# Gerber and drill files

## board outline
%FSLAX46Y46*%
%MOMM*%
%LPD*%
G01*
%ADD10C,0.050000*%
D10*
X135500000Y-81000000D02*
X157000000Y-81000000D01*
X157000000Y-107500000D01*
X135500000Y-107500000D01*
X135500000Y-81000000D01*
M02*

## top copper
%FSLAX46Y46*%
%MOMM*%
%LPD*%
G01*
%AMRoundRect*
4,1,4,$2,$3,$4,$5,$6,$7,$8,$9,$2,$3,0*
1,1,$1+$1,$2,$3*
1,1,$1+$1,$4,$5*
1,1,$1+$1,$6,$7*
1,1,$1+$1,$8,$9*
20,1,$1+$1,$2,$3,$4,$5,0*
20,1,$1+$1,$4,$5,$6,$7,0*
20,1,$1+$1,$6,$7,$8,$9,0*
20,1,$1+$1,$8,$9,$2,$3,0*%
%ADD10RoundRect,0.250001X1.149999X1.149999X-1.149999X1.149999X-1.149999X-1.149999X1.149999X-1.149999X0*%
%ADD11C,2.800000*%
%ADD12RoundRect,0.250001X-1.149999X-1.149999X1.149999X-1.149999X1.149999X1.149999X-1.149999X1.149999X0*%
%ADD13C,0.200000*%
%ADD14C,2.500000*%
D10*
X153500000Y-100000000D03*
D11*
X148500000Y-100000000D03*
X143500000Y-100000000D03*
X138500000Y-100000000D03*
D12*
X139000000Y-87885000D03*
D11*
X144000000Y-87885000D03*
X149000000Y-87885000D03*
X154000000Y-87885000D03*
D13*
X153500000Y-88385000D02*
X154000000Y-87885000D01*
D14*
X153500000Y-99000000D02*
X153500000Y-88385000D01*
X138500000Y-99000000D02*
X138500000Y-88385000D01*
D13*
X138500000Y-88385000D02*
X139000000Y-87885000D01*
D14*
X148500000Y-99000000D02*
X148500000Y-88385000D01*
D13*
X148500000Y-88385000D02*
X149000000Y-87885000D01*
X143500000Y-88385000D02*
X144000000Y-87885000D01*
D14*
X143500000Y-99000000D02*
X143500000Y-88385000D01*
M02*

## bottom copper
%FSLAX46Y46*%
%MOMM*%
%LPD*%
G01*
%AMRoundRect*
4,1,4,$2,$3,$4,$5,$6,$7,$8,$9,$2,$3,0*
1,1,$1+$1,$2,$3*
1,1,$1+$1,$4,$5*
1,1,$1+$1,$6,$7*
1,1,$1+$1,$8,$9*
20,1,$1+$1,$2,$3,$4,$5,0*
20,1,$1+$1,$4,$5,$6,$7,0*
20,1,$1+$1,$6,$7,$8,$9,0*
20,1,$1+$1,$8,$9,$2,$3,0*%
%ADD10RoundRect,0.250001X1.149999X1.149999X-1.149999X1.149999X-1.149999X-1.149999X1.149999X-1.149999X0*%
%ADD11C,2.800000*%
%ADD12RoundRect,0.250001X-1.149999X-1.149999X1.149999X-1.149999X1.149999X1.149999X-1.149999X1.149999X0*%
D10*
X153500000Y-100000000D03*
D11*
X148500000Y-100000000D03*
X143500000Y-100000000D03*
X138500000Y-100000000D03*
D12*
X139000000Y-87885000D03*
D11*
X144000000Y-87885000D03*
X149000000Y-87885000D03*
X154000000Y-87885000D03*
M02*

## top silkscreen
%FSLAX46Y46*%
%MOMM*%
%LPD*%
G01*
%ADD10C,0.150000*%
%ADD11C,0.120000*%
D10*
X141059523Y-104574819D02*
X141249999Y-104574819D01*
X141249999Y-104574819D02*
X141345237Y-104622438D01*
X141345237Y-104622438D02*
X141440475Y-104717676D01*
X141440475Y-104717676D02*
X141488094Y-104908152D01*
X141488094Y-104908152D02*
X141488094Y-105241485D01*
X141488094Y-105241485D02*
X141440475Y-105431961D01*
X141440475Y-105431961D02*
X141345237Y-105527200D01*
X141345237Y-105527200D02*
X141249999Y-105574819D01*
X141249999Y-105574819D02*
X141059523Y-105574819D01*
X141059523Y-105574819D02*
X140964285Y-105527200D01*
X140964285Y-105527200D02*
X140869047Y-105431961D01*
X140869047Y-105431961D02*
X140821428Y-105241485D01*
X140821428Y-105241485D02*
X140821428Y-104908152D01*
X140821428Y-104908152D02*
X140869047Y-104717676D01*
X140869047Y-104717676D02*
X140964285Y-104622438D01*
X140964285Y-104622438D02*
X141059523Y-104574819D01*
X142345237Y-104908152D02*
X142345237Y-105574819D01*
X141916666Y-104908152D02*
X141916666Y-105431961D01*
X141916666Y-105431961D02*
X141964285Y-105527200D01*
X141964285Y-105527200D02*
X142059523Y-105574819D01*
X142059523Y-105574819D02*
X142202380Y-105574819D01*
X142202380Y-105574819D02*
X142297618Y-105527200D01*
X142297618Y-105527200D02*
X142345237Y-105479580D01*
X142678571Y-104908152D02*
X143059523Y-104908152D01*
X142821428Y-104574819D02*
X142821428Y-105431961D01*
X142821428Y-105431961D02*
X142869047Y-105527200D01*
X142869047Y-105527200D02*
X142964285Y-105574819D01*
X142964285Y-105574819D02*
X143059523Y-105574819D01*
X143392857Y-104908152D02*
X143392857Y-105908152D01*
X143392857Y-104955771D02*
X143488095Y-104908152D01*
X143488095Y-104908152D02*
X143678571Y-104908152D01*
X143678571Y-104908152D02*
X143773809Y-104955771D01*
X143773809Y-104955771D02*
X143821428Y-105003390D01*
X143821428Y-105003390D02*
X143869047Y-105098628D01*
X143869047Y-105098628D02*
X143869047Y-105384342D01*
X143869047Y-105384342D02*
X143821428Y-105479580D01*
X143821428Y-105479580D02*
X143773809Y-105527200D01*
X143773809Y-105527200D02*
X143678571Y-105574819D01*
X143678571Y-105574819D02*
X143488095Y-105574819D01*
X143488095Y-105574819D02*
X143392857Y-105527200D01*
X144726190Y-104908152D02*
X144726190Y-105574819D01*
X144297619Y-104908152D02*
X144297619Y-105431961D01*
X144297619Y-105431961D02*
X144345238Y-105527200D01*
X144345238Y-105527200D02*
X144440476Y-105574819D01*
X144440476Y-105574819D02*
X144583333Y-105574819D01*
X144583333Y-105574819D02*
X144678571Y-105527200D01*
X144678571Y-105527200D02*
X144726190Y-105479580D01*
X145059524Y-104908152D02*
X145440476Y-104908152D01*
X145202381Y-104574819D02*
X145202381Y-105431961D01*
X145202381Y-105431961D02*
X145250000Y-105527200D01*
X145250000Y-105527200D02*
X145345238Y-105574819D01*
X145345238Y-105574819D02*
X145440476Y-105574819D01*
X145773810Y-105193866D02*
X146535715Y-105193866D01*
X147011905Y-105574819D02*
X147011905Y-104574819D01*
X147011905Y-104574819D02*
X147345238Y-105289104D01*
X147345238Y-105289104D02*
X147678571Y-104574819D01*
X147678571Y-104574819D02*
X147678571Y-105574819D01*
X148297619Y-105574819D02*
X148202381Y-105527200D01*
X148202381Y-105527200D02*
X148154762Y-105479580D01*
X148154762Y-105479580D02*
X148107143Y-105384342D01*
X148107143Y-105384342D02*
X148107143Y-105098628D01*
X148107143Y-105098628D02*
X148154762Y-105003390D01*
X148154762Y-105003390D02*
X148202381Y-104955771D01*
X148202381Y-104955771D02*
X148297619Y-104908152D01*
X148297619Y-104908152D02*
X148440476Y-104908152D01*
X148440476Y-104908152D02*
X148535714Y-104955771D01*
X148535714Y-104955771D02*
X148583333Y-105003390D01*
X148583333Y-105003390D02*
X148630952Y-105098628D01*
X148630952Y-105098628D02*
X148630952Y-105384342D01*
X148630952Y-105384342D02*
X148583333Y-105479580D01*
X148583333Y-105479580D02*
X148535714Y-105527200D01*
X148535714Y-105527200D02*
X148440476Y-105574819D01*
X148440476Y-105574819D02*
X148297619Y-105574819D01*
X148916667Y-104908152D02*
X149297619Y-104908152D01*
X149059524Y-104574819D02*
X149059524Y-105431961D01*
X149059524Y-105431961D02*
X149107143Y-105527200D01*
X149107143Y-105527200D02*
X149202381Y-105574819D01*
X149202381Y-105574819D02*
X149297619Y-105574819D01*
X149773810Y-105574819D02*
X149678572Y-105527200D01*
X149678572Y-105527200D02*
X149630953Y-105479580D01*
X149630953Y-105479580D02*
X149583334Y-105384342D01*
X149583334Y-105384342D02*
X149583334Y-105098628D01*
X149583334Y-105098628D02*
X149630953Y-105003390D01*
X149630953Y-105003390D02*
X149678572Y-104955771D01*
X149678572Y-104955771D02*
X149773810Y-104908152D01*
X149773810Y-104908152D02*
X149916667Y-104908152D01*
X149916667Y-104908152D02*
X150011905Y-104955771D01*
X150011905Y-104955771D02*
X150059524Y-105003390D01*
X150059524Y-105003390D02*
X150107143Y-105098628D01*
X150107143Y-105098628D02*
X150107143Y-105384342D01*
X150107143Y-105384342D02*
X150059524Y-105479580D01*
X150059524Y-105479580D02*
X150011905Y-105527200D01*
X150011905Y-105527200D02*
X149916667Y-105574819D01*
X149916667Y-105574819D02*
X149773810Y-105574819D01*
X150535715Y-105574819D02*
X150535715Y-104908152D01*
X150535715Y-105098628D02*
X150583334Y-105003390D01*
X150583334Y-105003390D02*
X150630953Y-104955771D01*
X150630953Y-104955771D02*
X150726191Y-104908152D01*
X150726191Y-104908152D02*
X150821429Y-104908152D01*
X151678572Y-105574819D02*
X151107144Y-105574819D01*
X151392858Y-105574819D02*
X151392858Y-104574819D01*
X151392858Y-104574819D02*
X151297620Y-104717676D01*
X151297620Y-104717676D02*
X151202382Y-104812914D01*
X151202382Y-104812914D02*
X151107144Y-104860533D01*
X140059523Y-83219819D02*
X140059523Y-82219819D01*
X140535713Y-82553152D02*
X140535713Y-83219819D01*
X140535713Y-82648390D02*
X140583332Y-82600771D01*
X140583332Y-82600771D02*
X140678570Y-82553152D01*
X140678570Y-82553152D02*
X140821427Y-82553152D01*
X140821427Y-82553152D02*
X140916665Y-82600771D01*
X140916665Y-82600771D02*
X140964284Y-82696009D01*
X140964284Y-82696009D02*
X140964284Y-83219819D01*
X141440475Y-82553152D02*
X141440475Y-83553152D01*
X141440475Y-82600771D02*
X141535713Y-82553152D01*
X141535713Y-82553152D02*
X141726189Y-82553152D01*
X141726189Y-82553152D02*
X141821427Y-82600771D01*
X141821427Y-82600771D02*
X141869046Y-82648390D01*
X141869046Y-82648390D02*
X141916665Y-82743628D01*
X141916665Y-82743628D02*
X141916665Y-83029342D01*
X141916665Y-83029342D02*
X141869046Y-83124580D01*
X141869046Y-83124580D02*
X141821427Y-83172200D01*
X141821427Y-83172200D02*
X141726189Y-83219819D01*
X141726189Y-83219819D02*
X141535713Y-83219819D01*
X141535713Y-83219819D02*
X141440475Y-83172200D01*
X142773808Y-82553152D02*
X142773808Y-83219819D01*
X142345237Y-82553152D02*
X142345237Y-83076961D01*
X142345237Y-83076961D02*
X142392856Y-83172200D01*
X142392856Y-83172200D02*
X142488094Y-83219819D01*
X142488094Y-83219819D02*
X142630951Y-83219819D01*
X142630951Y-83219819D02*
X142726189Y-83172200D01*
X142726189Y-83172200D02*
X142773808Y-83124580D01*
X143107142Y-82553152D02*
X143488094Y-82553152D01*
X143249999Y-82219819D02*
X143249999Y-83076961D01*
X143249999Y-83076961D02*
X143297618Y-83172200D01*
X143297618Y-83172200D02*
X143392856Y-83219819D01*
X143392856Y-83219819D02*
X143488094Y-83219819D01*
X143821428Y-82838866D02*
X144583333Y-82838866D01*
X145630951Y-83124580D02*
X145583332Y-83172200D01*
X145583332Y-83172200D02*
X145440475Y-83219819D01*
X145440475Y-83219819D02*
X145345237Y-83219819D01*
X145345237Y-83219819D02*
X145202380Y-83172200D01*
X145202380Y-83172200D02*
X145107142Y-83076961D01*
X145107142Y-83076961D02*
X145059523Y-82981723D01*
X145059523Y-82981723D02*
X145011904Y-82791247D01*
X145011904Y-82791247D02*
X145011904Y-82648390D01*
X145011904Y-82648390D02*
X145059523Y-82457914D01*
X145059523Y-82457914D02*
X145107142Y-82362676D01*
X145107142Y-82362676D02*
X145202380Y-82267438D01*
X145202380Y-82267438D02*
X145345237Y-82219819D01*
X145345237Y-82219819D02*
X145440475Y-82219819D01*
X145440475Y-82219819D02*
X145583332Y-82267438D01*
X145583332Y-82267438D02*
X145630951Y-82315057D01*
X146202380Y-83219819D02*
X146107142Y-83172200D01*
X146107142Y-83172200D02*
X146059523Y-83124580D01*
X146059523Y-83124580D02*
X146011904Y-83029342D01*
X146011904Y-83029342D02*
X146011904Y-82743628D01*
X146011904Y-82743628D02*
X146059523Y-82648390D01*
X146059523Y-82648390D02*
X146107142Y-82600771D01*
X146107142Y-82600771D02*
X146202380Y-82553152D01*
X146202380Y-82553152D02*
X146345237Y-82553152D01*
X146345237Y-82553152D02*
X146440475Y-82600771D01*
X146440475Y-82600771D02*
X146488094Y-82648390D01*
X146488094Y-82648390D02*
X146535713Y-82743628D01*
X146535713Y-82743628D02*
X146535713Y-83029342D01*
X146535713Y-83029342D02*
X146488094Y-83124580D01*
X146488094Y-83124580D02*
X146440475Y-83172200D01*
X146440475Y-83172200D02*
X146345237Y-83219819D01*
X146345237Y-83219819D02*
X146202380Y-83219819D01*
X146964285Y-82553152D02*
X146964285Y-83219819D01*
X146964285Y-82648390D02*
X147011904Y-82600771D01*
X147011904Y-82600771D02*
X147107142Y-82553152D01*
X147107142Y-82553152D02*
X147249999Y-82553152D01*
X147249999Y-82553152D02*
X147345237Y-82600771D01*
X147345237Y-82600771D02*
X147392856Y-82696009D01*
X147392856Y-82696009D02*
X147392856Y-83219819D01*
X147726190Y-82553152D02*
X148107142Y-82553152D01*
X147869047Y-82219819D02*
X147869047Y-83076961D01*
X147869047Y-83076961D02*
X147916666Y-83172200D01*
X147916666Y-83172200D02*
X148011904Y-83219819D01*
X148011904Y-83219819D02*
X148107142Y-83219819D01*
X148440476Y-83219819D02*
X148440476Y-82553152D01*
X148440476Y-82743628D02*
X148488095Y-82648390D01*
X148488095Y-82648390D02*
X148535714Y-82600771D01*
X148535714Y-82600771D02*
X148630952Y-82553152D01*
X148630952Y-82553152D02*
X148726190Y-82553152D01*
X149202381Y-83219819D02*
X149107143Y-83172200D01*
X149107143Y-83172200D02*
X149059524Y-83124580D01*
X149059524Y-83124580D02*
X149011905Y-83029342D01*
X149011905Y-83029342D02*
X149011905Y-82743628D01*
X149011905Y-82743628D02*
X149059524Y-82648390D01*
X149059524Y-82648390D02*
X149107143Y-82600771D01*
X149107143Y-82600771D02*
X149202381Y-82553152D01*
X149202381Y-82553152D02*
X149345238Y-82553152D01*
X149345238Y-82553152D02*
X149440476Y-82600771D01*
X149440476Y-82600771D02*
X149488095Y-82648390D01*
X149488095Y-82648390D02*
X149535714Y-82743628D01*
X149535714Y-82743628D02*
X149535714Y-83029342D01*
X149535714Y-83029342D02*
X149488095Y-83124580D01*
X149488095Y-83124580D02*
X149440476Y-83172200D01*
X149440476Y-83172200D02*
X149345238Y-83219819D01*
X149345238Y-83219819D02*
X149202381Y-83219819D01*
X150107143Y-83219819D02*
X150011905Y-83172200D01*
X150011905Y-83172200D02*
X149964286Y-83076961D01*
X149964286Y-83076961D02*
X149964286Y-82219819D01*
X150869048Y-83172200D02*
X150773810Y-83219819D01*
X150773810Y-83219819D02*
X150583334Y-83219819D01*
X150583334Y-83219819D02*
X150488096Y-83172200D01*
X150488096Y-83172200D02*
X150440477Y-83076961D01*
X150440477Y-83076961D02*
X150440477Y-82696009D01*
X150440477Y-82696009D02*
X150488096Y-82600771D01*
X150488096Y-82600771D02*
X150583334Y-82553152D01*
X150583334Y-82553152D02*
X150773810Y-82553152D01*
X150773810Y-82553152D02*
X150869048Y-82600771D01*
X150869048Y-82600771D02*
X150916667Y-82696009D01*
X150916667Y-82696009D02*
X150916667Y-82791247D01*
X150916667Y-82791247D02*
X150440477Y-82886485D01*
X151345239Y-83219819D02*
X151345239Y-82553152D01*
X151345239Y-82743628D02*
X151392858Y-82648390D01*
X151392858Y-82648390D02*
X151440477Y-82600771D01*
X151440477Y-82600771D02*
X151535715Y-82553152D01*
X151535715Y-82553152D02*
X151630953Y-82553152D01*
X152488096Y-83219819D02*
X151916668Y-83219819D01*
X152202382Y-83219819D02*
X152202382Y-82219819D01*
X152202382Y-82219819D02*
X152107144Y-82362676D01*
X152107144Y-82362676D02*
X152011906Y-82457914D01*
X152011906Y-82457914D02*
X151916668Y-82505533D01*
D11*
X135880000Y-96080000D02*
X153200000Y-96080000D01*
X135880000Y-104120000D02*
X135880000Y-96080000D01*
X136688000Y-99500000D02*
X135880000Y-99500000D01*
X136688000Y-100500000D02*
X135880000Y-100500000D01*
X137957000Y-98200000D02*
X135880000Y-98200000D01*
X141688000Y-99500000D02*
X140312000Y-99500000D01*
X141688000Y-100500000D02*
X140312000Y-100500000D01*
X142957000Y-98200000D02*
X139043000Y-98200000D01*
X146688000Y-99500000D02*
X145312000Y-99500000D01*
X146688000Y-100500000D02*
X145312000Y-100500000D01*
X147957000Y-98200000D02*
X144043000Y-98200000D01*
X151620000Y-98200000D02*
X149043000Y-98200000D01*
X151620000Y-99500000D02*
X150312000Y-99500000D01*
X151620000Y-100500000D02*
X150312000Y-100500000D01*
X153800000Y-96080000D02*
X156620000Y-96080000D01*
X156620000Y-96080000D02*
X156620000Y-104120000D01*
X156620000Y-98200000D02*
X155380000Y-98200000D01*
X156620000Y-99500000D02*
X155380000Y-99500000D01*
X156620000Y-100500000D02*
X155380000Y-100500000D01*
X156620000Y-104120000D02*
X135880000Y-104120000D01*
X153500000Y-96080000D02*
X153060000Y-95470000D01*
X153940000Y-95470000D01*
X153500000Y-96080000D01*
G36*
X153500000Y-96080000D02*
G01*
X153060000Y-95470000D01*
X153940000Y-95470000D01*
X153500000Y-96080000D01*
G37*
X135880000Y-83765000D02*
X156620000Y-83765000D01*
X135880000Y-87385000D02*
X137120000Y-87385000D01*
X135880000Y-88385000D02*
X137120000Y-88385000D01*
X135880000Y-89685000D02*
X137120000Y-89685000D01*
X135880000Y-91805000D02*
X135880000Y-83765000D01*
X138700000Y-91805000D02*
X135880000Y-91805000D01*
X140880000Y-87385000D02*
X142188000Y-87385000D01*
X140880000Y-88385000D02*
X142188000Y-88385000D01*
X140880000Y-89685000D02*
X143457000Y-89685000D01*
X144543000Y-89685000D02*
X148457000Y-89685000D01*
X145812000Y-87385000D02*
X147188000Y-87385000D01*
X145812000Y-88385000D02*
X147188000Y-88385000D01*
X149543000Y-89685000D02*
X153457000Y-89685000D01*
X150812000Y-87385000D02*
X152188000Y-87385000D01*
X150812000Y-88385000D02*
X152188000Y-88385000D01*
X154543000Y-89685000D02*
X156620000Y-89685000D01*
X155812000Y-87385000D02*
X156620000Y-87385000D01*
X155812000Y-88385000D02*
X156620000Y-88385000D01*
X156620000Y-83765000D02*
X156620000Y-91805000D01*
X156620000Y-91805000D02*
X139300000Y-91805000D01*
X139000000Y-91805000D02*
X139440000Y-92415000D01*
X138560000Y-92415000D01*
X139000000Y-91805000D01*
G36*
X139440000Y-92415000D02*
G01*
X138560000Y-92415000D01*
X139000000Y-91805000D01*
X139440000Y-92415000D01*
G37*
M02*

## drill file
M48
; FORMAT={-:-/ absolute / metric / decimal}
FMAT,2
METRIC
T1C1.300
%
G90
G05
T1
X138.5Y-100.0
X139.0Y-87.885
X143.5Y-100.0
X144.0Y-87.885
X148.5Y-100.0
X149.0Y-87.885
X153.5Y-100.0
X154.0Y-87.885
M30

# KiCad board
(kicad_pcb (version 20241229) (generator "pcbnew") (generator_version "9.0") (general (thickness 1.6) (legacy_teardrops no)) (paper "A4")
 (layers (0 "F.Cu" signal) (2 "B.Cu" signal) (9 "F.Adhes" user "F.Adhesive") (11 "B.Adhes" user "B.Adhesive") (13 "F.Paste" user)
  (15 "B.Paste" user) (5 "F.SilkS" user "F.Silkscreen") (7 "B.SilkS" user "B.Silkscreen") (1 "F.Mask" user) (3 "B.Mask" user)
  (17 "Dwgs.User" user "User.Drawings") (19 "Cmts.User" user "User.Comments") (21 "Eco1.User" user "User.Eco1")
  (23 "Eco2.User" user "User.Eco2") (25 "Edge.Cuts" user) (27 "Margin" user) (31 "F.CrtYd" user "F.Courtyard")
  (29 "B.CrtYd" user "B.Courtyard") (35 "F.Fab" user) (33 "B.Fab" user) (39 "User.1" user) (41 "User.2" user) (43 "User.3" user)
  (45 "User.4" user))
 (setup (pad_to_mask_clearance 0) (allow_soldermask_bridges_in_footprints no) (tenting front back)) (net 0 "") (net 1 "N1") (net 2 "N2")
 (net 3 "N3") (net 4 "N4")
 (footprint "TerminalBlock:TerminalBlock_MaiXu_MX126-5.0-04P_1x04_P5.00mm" (layer "F.Cu") (at 153.5 100 180)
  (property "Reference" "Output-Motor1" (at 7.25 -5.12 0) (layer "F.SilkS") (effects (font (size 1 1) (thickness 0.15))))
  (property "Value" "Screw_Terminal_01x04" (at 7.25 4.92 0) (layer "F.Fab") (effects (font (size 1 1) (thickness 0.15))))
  (fp_line (start 17.62 3.92) (end 0.3 3.92) (stroke (width 0.12) (type solid)) (layer "F.SilkS"))
  (fp_line (start 17.62 -4.12) (end 17.62 3.92) (stroke (width 0.12) (type solid)) (layer "F.SilkS"))
  (fp_line (start 16.812 0.5) (end 17.62 0.5) (stroke (width 0.12) (type solid)) (layer "F.SilkS"))
  (fp_line (start 16.812 -0.5) (end 17.62 -0.5) (stroke (width 0.12) (type solid)) (layer "F.SilkS"))
  (fp_line (start 15.543 1.8) (end 17.62 1.8) (stroke (width 0.12) (type solid)) (layer "F.SilkS"))
  (fp_line (start 11.812 0.5) (end 13.188 0.5) (stroke (width 0.12) (type solid)) (layer "F.SilkS"))
  (fp_line (start 11.812 -0.5) (end 13.188 -0.5) (stroke (width 0.12) (type solid)) (layer "F.SilkS"))
  (fp_line (start 10.543 1.8) (end 14.457 1.8) (stroke (width 0.12) (type solid)) (layer "F.SilkS"))
  (fp_line (start 6.812 0.5) (end 8.188 0.5) (stroke (width 0.12) (type solid)) (layer "F.SilkS"))
  (fp_line (start 6.812 -0.5) (end 8.188 -0.5) (stroke (width 0.12) (type solid)) (layer "F.SilkS"))
  (fp_line (start 5.543 1.8) (end 9.457 1.8) (stroke (width 0.12) (type solid)) (layer "F.SilkS"))
  (fp_line (start 1.88 1.8) (end 4.457 1.8) (stroke (width 0.12) (type solid)) (layer "F.SilkS"))
  (fp_line (start 1.88 0.5) (end 3.188 0.5) (stroke (width 0.12) (type solid)) (layer "F.SilkS"))
  (fp_line (start 1.88 -0.5) (end 3.188 -0.5) (stroke (width 0.12) (type solid)) (layer "F.SilkS"))
  (fp_line (start -0.3 3.92) (end -3.12 3.92) (stroke (width 0.12) (type solid)) (layer "F.SilkS"))
  (fp_line (start -3.12 3.92) (end -3.12 -4.12) (stroke (width 0.12) (type solid)) (layer "F.SilkS"))
  (fp_line (start -3.12 1.8) (end -1.88 1.8) (stroke (width 0.12) (type solid)) (layer "F.SilkS"))
  (fp_line (start -3.12 0.5) (end -1.88 0.5) (stroke (width 0.12) (type solid)) (layer "F.SilkS"))
  (fp_line (start -3.12 -0.5) (end -1.88 -0.5) (stroke (width 0.12) (type solid)) (layer "F.SilkS"))
  (fp_line (start -3.12 -4.12) (end 17.62 -4.12) (stroke (width 0.12) (type solid)) (layer "F.SilkS"))
  (fp_poly (pts (xy 0 3.92) (xy 0.44 4.53) (xy -0.44 4.53)) (stroke (width 0.12) (type solid)) (fill yes) (layer "F.SilkS"))
  (pad "1" thru_hole roundrect (at 0 0 180) (size 2.8 2.8) (drill 1.3) (layers "*.Cu" "*.Mask") (remove_unused_layers no)
   (roundrect_rratio 0.089286) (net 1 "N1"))
  (pad "2" thru_hole circle (at 5 0 180) (size 2.8 2.8) (drill 1.3) (layers "*.Cu" "*.Mask") (remove_unused_layers no) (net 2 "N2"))
  (pad "3" thru_hole circle (at 10 0 180) (size 2.8 2.8) (drill 1.3) (layers "*.Cu" "*.Mask") (remove_unused_layers no) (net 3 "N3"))
  (pad "4" thru_hole circle (at 15 0 180) (size 2.8 2.8) (drill 1.3) (layers "*.Cu" "*.Mask") (remove_unused_layers no) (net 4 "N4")))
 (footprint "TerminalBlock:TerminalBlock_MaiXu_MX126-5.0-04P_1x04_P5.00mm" (layer "F.Cu") (at 139 87.885)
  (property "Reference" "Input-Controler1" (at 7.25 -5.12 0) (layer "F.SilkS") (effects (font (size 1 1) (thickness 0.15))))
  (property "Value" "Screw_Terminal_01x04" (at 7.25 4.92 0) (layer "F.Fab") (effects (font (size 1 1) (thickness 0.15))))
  (fp_line (start -3.12 -4.12) (end 17.62 -4.12) (stroke (width 0.12) (type solid)) (layer "F.SilkS"))
  (fp_line (start -3.12 -0.5) (end -1.88 -0.5) (stroke (width 0.12) (type solid)) (layer "F.SilkS"))
  (fp_line (start -3.12 0.5) (end -1.88 0.5) (stroke (width 0.12) (type solid)) (layer "F.SilkS"))
  (fp_line (start -3.12 1.8) (end -1.88 1.8) (stroke (width 0.12) (type solid)) (layer "F.SilkS"))
  (fp_line (start -3.12 3.92) (end -3.12 -4.12) (stroke (width 0.12) (type solid)) (layer "F.SilkS"))
  (fp_line (start -0.3 3.92) (end -3.12 3.92) (stroke (width 0.12) (type solid)) (layer "F.SilkS"))
  (fp_line (start 1.88 -0.5) (end 3.188 -0.5) (stroke (width 0.12) (type solid)) (layer "F.SilkS"))
  (fp_line (start 1.88 0.5) (end 3.188 0.5) (stroke (width 0.12) (type solid)) (layer "F.SilkS"))
  (fp_line (start 1.88 1.8) (end 4.457 1.8) (stroke (width 0.12) (type solid)) (layer "F.SilkS"))
  (fp_line (start 5.543 1.8) (end 9.457 1.8) (stroke (width 0.12) (type solid)) (layer "F.SilkS"))
  (fp_line (start 6.812 -0.5) (end 8.188 -0.5) (stroke (width 0.12) (type solid)) (layer "F.SilkS"))
  (fp_line (start 6.812 0.5) (end 8.188 0.5) (stroke (width 0.12) (type solid)) (layer "F.SilkS"))
  (fp_line (start 10.543 1.8) (end 14.457 1.8) (stroke (width 0.12) (type solid)) (layer "F.SilkS"))
  (fp_line (start 11.812 -0.5) (end 13.188 -0.5) (stroke (width 0.12) (type solid)) (layer "F.SilkS"))
  (fp_line (start 11.812 0.5) (end 13.188 0.5) (stroke (width 0.12) (type solid)) (layer "F.SilkS"))
  (fp_line (start 15.543 1.8) (end 17.62 1.8) (stroke (width 0.12) (type solid)) (layer "F.SilkS"))
  (fp_line (start 16.812 -0.5) (end 17.62 -0.5) (stroke (width 0.12) (type solid)) (layer "F.SilkS"))
  (fp_line (start 16.812 0.5) (end 17.62 0.5) (stroke (width 0.12) (type solid)) (layer "F.SilkS"))
  (fp_line (start 17.62 -4.12) (end 17.62 3.92) (stroke (width 0.12) (type solid)) (layer "F.SilkS"))
  (fp_line (start 17.62 3.92) (end 0.3 3.92) (stroke (width 0.12) (type solid)) (layer "F.SilkS"))
  (fp_poly (pts (xy 0 3.92) (xy 0.44 4.53) (xy -0.44 4.53)) (stroke (width 0.12) (type solid)) (fill yes) (layer "F.SilkS"))
  (pad "1" thru_hole roundrect (at 0 0) (size 2.8 2.8) (drill 1.3) (layers "*.Cu" "*.Mask") (remove_unused_layers no)
   (roundrect_rratio 0.089286) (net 4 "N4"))
  (pad "2" thru_hole circle (at 5 0) (size 2.8 2.8) (drill 1.3) (layers "*.Cu" "*.Mask") (remove_unused_layers no) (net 3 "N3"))
  (pad "3" thru_hole circle (at 10 0) (size 2.8 2.8) (drill 1.3) (layers "*.Cu" "*.Mask") (remove_unused_layers no) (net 2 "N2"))
  (pad "4" thru_hole circle (at 15 0) (size 2.8 2.8) (drill 1.3) (layers "*.Cu" "*.Mask") (remove_unused_layers no) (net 1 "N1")))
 (gr_rect (start 135.5 81) (end 157 107.5) (stroke (width 0.05) (type default)) (fill no) (layer "Edge.Cuts"))
 (segment (start 153.5 88.385) (end 154 87.885) (width 0.2) (layer "F.Cu") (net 1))
 (segment (start 153.5 99) (end 153.5 88.385) (width 2.5) (layer "F.Cu") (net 1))
 (segment (start 138.5 99) (end 138.5 88.385) (width 2.5) (layer "F.Cu") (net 4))
 (segment (start 138.5 88.385) (end 139 87.885) (width 0.2) (layer "F.Cu") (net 4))
 (segment (start 148.5 99) (end 148.5 88.385) (width 2.5) (layer "F.Cu") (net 2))
 (segment (start 148.5 88.385) (end 149 87.885) (width 0.2) (layer "F.Cu") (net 2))
 (segment (start 143.5 88.385) (end 144 87.885) (width 0.2) (layer "F.Cu") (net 3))
 (segment (start 143.5 99) (end 143.5 88.385) (width 2.5) (layer "F.Cu") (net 3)))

